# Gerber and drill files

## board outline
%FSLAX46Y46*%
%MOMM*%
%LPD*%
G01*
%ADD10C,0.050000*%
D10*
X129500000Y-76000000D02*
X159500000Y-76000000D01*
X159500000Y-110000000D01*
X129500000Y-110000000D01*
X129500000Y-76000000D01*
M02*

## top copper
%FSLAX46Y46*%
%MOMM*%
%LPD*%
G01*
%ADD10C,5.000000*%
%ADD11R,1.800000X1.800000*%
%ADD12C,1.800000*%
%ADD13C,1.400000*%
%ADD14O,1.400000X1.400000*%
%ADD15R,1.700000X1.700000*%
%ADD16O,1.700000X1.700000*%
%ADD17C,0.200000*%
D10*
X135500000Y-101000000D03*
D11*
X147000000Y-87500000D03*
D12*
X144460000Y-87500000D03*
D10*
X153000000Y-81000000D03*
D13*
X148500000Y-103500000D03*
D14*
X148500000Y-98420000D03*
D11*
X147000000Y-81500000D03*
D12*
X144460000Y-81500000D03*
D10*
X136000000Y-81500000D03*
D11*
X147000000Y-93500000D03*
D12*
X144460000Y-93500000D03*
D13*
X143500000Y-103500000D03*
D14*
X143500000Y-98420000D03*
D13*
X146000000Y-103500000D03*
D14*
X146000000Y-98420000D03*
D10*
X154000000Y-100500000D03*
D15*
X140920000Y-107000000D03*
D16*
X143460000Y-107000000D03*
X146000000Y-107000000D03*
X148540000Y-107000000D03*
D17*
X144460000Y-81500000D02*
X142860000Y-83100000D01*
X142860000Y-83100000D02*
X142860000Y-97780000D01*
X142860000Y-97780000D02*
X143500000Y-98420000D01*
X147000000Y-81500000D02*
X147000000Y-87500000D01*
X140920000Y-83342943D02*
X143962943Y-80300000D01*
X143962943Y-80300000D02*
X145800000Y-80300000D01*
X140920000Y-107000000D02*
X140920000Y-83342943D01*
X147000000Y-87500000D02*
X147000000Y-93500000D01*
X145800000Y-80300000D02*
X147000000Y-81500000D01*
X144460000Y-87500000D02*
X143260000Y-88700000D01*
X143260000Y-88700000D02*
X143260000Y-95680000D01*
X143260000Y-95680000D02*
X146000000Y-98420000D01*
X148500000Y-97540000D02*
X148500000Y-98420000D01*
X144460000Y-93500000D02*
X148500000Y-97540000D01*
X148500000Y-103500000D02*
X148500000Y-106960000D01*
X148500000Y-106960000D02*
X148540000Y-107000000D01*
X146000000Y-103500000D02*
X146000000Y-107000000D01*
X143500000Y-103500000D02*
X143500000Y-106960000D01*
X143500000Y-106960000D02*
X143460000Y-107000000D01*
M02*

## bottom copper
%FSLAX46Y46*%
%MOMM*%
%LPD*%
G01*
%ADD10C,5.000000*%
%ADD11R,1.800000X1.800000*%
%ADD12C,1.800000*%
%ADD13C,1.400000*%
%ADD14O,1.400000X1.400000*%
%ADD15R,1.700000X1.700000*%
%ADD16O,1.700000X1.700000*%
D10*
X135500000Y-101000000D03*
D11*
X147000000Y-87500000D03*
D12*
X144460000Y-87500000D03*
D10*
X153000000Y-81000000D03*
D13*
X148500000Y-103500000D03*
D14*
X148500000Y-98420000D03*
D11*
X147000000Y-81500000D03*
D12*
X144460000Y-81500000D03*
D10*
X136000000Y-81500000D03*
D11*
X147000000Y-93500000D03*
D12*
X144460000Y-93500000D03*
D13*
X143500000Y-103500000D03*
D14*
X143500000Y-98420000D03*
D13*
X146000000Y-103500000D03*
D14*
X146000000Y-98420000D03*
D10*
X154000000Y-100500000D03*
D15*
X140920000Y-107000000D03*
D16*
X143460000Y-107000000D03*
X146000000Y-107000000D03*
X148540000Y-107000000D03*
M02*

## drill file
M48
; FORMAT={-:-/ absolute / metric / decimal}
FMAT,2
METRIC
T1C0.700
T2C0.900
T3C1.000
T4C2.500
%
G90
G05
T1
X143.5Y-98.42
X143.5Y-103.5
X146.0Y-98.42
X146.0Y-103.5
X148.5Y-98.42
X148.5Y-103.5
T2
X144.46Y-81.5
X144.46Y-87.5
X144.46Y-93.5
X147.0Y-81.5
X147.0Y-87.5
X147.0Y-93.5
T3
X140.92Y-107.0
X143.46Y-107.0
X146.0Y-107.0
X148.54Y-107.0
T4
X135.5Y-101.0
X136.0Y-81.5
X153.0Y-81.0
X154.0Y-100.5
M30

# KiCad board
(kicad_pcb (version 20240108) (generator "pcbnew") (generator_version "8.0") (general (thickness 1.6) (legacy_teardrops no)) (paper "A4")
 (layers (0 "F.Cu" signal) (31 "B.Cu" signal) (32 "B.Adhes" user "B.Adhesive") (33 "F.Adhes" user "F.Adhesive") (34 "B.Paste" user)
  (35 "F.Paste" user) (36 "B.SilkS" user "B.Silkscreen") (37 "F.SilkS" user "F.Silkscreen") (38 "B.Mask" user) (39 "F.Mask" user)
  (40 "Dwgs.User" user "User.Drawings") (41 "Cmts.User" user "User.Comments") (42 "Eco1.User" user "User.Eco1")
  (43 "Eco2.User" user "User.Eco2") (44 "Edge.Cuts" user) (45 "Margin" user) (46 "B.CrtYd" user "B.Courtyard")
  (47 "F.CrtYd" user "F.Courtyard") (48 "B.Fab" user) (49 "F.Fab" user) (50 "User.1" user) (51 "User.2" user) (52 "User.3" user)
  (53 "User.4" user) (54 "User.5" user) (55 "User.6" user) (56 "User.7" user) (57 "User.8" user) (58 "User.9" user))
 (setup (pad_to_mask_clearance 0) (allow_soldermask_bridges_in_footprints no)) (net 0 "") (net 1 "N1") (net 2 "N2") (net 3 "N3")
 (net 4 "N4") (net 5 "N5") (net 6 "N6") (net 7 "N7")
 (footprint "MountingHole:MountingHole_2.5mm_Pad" (layer "F.Cu") (at 135.5 101)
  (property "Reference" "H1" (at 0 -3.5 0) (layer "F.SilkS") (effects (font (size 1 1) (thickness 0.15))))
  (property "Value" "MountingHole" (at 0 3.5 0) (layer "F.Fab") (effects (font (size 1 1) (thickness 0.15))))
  (pad "1" thru_hole circle (at 0 0) (size 5 5) (drill 2.5) (layers "*.Cu" "*.Mask") (remove_unused_layers no)))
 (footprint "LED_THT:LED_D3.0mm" (layer "F.Cu") (at 147 87.5 180)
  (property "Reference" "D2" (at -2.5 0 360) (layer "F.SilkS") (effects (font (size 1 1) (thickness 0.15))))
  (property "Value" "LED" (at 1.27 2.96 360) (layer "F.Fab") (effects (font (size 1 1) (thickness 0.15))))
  (pad "1" thru_hole rect (at 0 0 180) (size 1.8 1.8) (drill 0.9) (layers "*.Cu" "*.Mask") (remove_unused_layers no) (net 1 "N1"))
  (pad "2" thru_hole circle (at 2.54 0 180) (size 1.8 1.8) (drill 0.9) (layers "*.Cu" "*.Mask") (remove_unused_layers no) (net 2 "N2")))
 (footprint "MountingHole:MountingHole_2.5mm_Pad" (layer "F.Cu") (at 153 81)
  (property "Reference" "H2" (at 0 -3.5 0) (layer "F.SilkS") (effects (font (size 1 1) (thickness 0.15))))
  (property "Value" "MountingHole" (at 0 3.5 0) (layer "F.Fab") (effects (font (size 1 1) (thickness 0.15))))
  (pad "1" thru_hole circle (at 0 0) (size 5 5) (drill 2.5) (layers "*.Cu" "*.Mask") (remove_unused_layers no)))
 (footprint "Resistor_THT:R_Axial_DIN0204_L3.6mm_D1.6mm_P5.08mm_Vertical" (layer "F.Cu") (at 148.5 103.5 90)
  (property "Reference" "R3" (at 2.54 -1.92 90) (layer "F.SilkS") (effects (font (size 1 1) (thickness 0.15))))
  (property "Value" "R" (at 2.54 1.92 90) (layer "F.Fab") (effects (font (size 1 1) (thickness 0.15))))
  (pad "1" thru_hole circle (at 0 0 90) (size 1.4 1.4) (drill 0.7) (layers "*.Cu" "*.Mask") (remove_unused_layers no) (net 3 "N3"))
  (pad "2" thru_hole oval (at 5.08 0 90) (size 1.4 1.4) (drill 0.7) (layers "*.Cu" "*.Mask") (remove_unused_layers no) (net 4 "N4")))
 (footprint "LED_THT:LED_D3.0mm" (layer "F.Cu") (at 147 81.5 180)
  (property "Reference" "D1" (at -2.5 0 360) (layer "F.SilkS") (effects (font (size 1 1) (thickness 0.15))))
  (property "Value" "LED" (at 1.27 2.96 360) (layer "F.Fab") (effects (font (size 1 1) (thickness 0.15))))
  (pad "1" thru_hole rect (at 0 0 180) (size 1.8 1.8) (drill 0.9) (layers "*.Cu" "*.Mask") (remove_unused_layers no) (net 1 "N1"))
  (pad "2" thru_hole circle (at 2.54 0 180) (size 1.8 1.8) (drill 0.9) (layers "*.Cu" "*.Mask") (remove_unused_layers no) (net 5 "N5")))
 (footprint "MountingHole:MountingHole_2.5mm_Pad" (layer "F.Cu") (at 136 81.5)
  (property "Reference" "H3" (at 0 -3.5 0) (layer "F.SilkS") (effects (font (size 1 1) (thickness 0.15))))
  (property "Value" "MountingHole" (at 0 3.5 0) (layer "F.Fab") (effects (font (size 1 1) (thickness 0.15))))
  (pad "1" thru_hole circle (at 0 0) (size 5 5) (drill 2.5) (layers "*.Cu" "*.Mask") (remove_unused_layers no)))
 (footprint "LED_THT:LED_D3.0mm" (layer "F.Cu") (at 147 93.5 180)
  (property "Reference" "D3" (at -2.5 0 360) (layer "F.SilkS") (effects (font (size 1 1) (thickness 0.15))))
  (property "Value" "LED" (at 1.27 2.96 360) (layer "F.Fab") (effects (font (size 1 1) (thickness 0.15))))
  (pad "1" thru_hole rect (at 0 0 180) (size 1.8 1.8) (drill 0.9) (layers "*.Cu" "*.Mask") (remove_unused_layers no) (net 1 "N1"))
  (pad "2" thru_hole circle (at 2.54 0 180) (size 1.8 1.8) (drill 0.9) (layers "*.Cu" "*.Mask") (remove_unused_layers no) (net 4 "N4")))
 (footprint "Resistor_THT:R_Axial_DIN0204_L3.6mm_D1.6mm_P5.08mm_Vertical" (layer "F.Cu") (at 143.5 103.5 90)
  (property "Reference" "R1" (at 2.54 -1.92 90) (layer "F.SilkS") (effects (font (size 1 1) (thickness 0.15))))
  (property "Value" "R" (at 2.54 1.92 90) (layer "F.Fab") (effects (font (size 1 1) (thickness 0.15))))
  (pad "1" thru_hole circle (at 0 0 90) (size 1.4 1.4) (drill 0.7) (layers "*.Cu" "*.Mask") (remove_unused_layers no) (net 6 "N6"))
  (pad "2" thru_hole oval (at 5.08 0 90) (size 1.4 1.4) (drill 0.7) (layers "*.Cu" "*.Mask") (remove_unused_layers no) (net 5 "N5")))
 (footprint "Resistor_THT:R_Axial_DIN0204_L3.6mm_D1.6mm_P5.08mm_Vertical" (layer "F.Cu") (at 146 103.5 90)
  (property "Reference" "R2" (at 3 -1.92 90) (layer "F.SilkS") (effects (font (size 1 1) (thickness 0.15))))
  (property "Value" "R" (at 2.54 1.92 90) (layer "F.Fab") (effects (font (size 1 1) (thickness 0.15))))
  (pad "1" thru_hole circle (at 0 0 90) (size 1.4 1.4) (drill 0.7) (layers "*.Cu" "*.Mask") (remove_unused_layers no) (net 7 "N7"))
  (pad "2" thru_hole oval (at 5.08 0 90) (size 1.4 1.4) (drill 0.7) (layers "*.Cu" "*.Mask") (remove_unused_layers no) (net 2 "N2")))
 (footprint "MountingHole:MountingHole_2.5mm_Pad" (layer "F.Cu") (at 154 100.5)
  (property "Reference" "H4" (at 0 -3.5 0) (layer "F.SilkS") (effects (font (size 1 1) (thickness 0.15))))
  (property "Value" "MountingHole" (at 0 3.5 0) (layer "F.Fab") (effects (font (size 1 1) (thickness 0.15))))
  (pad "1" thru_hole circle (at 0 0) (size 5 5) (drill 2.5) (layers "*.Cu" "*.Mask") (remove_unused_layers no)))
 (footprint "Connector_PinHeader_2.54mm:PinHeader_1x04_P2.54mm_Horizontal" (layer "B.Cu") (at 140.92 107 -90)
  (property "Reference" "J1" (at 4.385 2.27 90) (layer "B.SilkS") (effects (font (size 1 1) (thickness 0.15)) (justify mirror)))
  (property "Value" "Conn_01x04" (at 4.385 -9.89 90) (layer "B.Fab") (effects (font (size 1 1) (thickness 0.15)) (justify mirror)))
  (pad "1" thru_hole rect (at 0 0 270) (size 1.7 1.7) (drill 1) (layers "*.Cu" "*.Mask") (remove_unused_layers no) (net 1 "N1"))
  (pad "2" thru_hole oval (at 0 -2.54 270) (size 1.7 1.7) (drill 1) (layers "*.Cu" "*.Mask") (remove_unused_layers no) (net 6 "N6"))
  (pad "3" thru_hole oval (at 0 -5.08 270) (size 1.7 1.7) (drill 1) (layers "*.Cu" "*.Mask") (remove_unused_layers no) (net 7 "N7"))
  (pad "4" thru_hole oval (at 0 -7.62 270) (size 1.7 1.7) (drill 1) (layers "*.Cu" "*.Mask") (remove_unused_layers no) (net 3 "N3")))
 (gr_rect (start 129.5 76) (end 159.5 110) (stroke (width 0.05) (type default)) (fill none) (layer "Edge.Cuts"))
 (segment (start 144.46 81.5) (end 142.86 83.1) (width 0.2) (layer "F.Cu") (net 5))
 (segment (start 142.86 83.1) (end 142.86 97.78) (width 0.2) (layer "F.Cu") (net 5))
 (segment (start 142.86 97.78) (end 143.5 98.42) (width 0.2) (layer "F.Cu") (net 5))
 (segment (start 147 81.5) (end 147 87.5) (width 0.2) (layer "F.Cu") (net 1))
 (segment (start 140.92 83.342943) (end 143.962943 80.3) (width 0.2) (layer "F.Cu") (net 1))
 (segment (start 143.962943 80.3) (end 145.8 80.3) (width 0.2) (layer "F.Cu") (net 1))
 (segment (start 140.92 107) (end 140.92 83.342943) (width 0.2) (layer "F.Cu") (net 1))
 (segment (start 147 87.5) (end 147 93.5) (width 0.2) (layer "F.Cu") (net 1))
 (segment (start 145.8 80.3) (end 147 81.5) (width 0.2) (layer "F.Cu") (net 1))
 (segment (start 144.46 87.5) (end 143.26 88.7) (width 0.2) (layer "F.Cu") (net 2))
 (segment (start 143.26 88.7) (end 143.26 95.68) (width 0.2) (layer "F.Cu") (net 2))
 (segment (start 143.26 95.68) (end 146 98.42) (width 0.2) (layer "F.Cu") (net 2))
 (segment (start 148.5 97.54) (end 148.5 98.42) (width 0.2) (layer "F.Cu") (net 4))
 (segment (start 144.46 93.5) (end 148.5 97.54) (width 0.2) (layer "F.Cu") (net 4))
 (segment (start 148.5 103.5) (end 148.5 106.96) (width 0.2) (layer "F.Cu") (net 3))
 (segment (start 148.5 106.96) (end 148.54 107) (width 0.2) (layer "F.Cu") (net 3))
 (segment (start 146 103.5) (end 146 107) (width 0.2) (layer "F.Cu") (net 7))
 (segment (start 143.5 103.5) (end 143.5 106.96) (width 0.2) (layer "F.Cu") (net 6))
 (segment (start 143.5 106.96) (end 143.46 107) (width 0.2) (layer "F.Cu") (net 6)))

